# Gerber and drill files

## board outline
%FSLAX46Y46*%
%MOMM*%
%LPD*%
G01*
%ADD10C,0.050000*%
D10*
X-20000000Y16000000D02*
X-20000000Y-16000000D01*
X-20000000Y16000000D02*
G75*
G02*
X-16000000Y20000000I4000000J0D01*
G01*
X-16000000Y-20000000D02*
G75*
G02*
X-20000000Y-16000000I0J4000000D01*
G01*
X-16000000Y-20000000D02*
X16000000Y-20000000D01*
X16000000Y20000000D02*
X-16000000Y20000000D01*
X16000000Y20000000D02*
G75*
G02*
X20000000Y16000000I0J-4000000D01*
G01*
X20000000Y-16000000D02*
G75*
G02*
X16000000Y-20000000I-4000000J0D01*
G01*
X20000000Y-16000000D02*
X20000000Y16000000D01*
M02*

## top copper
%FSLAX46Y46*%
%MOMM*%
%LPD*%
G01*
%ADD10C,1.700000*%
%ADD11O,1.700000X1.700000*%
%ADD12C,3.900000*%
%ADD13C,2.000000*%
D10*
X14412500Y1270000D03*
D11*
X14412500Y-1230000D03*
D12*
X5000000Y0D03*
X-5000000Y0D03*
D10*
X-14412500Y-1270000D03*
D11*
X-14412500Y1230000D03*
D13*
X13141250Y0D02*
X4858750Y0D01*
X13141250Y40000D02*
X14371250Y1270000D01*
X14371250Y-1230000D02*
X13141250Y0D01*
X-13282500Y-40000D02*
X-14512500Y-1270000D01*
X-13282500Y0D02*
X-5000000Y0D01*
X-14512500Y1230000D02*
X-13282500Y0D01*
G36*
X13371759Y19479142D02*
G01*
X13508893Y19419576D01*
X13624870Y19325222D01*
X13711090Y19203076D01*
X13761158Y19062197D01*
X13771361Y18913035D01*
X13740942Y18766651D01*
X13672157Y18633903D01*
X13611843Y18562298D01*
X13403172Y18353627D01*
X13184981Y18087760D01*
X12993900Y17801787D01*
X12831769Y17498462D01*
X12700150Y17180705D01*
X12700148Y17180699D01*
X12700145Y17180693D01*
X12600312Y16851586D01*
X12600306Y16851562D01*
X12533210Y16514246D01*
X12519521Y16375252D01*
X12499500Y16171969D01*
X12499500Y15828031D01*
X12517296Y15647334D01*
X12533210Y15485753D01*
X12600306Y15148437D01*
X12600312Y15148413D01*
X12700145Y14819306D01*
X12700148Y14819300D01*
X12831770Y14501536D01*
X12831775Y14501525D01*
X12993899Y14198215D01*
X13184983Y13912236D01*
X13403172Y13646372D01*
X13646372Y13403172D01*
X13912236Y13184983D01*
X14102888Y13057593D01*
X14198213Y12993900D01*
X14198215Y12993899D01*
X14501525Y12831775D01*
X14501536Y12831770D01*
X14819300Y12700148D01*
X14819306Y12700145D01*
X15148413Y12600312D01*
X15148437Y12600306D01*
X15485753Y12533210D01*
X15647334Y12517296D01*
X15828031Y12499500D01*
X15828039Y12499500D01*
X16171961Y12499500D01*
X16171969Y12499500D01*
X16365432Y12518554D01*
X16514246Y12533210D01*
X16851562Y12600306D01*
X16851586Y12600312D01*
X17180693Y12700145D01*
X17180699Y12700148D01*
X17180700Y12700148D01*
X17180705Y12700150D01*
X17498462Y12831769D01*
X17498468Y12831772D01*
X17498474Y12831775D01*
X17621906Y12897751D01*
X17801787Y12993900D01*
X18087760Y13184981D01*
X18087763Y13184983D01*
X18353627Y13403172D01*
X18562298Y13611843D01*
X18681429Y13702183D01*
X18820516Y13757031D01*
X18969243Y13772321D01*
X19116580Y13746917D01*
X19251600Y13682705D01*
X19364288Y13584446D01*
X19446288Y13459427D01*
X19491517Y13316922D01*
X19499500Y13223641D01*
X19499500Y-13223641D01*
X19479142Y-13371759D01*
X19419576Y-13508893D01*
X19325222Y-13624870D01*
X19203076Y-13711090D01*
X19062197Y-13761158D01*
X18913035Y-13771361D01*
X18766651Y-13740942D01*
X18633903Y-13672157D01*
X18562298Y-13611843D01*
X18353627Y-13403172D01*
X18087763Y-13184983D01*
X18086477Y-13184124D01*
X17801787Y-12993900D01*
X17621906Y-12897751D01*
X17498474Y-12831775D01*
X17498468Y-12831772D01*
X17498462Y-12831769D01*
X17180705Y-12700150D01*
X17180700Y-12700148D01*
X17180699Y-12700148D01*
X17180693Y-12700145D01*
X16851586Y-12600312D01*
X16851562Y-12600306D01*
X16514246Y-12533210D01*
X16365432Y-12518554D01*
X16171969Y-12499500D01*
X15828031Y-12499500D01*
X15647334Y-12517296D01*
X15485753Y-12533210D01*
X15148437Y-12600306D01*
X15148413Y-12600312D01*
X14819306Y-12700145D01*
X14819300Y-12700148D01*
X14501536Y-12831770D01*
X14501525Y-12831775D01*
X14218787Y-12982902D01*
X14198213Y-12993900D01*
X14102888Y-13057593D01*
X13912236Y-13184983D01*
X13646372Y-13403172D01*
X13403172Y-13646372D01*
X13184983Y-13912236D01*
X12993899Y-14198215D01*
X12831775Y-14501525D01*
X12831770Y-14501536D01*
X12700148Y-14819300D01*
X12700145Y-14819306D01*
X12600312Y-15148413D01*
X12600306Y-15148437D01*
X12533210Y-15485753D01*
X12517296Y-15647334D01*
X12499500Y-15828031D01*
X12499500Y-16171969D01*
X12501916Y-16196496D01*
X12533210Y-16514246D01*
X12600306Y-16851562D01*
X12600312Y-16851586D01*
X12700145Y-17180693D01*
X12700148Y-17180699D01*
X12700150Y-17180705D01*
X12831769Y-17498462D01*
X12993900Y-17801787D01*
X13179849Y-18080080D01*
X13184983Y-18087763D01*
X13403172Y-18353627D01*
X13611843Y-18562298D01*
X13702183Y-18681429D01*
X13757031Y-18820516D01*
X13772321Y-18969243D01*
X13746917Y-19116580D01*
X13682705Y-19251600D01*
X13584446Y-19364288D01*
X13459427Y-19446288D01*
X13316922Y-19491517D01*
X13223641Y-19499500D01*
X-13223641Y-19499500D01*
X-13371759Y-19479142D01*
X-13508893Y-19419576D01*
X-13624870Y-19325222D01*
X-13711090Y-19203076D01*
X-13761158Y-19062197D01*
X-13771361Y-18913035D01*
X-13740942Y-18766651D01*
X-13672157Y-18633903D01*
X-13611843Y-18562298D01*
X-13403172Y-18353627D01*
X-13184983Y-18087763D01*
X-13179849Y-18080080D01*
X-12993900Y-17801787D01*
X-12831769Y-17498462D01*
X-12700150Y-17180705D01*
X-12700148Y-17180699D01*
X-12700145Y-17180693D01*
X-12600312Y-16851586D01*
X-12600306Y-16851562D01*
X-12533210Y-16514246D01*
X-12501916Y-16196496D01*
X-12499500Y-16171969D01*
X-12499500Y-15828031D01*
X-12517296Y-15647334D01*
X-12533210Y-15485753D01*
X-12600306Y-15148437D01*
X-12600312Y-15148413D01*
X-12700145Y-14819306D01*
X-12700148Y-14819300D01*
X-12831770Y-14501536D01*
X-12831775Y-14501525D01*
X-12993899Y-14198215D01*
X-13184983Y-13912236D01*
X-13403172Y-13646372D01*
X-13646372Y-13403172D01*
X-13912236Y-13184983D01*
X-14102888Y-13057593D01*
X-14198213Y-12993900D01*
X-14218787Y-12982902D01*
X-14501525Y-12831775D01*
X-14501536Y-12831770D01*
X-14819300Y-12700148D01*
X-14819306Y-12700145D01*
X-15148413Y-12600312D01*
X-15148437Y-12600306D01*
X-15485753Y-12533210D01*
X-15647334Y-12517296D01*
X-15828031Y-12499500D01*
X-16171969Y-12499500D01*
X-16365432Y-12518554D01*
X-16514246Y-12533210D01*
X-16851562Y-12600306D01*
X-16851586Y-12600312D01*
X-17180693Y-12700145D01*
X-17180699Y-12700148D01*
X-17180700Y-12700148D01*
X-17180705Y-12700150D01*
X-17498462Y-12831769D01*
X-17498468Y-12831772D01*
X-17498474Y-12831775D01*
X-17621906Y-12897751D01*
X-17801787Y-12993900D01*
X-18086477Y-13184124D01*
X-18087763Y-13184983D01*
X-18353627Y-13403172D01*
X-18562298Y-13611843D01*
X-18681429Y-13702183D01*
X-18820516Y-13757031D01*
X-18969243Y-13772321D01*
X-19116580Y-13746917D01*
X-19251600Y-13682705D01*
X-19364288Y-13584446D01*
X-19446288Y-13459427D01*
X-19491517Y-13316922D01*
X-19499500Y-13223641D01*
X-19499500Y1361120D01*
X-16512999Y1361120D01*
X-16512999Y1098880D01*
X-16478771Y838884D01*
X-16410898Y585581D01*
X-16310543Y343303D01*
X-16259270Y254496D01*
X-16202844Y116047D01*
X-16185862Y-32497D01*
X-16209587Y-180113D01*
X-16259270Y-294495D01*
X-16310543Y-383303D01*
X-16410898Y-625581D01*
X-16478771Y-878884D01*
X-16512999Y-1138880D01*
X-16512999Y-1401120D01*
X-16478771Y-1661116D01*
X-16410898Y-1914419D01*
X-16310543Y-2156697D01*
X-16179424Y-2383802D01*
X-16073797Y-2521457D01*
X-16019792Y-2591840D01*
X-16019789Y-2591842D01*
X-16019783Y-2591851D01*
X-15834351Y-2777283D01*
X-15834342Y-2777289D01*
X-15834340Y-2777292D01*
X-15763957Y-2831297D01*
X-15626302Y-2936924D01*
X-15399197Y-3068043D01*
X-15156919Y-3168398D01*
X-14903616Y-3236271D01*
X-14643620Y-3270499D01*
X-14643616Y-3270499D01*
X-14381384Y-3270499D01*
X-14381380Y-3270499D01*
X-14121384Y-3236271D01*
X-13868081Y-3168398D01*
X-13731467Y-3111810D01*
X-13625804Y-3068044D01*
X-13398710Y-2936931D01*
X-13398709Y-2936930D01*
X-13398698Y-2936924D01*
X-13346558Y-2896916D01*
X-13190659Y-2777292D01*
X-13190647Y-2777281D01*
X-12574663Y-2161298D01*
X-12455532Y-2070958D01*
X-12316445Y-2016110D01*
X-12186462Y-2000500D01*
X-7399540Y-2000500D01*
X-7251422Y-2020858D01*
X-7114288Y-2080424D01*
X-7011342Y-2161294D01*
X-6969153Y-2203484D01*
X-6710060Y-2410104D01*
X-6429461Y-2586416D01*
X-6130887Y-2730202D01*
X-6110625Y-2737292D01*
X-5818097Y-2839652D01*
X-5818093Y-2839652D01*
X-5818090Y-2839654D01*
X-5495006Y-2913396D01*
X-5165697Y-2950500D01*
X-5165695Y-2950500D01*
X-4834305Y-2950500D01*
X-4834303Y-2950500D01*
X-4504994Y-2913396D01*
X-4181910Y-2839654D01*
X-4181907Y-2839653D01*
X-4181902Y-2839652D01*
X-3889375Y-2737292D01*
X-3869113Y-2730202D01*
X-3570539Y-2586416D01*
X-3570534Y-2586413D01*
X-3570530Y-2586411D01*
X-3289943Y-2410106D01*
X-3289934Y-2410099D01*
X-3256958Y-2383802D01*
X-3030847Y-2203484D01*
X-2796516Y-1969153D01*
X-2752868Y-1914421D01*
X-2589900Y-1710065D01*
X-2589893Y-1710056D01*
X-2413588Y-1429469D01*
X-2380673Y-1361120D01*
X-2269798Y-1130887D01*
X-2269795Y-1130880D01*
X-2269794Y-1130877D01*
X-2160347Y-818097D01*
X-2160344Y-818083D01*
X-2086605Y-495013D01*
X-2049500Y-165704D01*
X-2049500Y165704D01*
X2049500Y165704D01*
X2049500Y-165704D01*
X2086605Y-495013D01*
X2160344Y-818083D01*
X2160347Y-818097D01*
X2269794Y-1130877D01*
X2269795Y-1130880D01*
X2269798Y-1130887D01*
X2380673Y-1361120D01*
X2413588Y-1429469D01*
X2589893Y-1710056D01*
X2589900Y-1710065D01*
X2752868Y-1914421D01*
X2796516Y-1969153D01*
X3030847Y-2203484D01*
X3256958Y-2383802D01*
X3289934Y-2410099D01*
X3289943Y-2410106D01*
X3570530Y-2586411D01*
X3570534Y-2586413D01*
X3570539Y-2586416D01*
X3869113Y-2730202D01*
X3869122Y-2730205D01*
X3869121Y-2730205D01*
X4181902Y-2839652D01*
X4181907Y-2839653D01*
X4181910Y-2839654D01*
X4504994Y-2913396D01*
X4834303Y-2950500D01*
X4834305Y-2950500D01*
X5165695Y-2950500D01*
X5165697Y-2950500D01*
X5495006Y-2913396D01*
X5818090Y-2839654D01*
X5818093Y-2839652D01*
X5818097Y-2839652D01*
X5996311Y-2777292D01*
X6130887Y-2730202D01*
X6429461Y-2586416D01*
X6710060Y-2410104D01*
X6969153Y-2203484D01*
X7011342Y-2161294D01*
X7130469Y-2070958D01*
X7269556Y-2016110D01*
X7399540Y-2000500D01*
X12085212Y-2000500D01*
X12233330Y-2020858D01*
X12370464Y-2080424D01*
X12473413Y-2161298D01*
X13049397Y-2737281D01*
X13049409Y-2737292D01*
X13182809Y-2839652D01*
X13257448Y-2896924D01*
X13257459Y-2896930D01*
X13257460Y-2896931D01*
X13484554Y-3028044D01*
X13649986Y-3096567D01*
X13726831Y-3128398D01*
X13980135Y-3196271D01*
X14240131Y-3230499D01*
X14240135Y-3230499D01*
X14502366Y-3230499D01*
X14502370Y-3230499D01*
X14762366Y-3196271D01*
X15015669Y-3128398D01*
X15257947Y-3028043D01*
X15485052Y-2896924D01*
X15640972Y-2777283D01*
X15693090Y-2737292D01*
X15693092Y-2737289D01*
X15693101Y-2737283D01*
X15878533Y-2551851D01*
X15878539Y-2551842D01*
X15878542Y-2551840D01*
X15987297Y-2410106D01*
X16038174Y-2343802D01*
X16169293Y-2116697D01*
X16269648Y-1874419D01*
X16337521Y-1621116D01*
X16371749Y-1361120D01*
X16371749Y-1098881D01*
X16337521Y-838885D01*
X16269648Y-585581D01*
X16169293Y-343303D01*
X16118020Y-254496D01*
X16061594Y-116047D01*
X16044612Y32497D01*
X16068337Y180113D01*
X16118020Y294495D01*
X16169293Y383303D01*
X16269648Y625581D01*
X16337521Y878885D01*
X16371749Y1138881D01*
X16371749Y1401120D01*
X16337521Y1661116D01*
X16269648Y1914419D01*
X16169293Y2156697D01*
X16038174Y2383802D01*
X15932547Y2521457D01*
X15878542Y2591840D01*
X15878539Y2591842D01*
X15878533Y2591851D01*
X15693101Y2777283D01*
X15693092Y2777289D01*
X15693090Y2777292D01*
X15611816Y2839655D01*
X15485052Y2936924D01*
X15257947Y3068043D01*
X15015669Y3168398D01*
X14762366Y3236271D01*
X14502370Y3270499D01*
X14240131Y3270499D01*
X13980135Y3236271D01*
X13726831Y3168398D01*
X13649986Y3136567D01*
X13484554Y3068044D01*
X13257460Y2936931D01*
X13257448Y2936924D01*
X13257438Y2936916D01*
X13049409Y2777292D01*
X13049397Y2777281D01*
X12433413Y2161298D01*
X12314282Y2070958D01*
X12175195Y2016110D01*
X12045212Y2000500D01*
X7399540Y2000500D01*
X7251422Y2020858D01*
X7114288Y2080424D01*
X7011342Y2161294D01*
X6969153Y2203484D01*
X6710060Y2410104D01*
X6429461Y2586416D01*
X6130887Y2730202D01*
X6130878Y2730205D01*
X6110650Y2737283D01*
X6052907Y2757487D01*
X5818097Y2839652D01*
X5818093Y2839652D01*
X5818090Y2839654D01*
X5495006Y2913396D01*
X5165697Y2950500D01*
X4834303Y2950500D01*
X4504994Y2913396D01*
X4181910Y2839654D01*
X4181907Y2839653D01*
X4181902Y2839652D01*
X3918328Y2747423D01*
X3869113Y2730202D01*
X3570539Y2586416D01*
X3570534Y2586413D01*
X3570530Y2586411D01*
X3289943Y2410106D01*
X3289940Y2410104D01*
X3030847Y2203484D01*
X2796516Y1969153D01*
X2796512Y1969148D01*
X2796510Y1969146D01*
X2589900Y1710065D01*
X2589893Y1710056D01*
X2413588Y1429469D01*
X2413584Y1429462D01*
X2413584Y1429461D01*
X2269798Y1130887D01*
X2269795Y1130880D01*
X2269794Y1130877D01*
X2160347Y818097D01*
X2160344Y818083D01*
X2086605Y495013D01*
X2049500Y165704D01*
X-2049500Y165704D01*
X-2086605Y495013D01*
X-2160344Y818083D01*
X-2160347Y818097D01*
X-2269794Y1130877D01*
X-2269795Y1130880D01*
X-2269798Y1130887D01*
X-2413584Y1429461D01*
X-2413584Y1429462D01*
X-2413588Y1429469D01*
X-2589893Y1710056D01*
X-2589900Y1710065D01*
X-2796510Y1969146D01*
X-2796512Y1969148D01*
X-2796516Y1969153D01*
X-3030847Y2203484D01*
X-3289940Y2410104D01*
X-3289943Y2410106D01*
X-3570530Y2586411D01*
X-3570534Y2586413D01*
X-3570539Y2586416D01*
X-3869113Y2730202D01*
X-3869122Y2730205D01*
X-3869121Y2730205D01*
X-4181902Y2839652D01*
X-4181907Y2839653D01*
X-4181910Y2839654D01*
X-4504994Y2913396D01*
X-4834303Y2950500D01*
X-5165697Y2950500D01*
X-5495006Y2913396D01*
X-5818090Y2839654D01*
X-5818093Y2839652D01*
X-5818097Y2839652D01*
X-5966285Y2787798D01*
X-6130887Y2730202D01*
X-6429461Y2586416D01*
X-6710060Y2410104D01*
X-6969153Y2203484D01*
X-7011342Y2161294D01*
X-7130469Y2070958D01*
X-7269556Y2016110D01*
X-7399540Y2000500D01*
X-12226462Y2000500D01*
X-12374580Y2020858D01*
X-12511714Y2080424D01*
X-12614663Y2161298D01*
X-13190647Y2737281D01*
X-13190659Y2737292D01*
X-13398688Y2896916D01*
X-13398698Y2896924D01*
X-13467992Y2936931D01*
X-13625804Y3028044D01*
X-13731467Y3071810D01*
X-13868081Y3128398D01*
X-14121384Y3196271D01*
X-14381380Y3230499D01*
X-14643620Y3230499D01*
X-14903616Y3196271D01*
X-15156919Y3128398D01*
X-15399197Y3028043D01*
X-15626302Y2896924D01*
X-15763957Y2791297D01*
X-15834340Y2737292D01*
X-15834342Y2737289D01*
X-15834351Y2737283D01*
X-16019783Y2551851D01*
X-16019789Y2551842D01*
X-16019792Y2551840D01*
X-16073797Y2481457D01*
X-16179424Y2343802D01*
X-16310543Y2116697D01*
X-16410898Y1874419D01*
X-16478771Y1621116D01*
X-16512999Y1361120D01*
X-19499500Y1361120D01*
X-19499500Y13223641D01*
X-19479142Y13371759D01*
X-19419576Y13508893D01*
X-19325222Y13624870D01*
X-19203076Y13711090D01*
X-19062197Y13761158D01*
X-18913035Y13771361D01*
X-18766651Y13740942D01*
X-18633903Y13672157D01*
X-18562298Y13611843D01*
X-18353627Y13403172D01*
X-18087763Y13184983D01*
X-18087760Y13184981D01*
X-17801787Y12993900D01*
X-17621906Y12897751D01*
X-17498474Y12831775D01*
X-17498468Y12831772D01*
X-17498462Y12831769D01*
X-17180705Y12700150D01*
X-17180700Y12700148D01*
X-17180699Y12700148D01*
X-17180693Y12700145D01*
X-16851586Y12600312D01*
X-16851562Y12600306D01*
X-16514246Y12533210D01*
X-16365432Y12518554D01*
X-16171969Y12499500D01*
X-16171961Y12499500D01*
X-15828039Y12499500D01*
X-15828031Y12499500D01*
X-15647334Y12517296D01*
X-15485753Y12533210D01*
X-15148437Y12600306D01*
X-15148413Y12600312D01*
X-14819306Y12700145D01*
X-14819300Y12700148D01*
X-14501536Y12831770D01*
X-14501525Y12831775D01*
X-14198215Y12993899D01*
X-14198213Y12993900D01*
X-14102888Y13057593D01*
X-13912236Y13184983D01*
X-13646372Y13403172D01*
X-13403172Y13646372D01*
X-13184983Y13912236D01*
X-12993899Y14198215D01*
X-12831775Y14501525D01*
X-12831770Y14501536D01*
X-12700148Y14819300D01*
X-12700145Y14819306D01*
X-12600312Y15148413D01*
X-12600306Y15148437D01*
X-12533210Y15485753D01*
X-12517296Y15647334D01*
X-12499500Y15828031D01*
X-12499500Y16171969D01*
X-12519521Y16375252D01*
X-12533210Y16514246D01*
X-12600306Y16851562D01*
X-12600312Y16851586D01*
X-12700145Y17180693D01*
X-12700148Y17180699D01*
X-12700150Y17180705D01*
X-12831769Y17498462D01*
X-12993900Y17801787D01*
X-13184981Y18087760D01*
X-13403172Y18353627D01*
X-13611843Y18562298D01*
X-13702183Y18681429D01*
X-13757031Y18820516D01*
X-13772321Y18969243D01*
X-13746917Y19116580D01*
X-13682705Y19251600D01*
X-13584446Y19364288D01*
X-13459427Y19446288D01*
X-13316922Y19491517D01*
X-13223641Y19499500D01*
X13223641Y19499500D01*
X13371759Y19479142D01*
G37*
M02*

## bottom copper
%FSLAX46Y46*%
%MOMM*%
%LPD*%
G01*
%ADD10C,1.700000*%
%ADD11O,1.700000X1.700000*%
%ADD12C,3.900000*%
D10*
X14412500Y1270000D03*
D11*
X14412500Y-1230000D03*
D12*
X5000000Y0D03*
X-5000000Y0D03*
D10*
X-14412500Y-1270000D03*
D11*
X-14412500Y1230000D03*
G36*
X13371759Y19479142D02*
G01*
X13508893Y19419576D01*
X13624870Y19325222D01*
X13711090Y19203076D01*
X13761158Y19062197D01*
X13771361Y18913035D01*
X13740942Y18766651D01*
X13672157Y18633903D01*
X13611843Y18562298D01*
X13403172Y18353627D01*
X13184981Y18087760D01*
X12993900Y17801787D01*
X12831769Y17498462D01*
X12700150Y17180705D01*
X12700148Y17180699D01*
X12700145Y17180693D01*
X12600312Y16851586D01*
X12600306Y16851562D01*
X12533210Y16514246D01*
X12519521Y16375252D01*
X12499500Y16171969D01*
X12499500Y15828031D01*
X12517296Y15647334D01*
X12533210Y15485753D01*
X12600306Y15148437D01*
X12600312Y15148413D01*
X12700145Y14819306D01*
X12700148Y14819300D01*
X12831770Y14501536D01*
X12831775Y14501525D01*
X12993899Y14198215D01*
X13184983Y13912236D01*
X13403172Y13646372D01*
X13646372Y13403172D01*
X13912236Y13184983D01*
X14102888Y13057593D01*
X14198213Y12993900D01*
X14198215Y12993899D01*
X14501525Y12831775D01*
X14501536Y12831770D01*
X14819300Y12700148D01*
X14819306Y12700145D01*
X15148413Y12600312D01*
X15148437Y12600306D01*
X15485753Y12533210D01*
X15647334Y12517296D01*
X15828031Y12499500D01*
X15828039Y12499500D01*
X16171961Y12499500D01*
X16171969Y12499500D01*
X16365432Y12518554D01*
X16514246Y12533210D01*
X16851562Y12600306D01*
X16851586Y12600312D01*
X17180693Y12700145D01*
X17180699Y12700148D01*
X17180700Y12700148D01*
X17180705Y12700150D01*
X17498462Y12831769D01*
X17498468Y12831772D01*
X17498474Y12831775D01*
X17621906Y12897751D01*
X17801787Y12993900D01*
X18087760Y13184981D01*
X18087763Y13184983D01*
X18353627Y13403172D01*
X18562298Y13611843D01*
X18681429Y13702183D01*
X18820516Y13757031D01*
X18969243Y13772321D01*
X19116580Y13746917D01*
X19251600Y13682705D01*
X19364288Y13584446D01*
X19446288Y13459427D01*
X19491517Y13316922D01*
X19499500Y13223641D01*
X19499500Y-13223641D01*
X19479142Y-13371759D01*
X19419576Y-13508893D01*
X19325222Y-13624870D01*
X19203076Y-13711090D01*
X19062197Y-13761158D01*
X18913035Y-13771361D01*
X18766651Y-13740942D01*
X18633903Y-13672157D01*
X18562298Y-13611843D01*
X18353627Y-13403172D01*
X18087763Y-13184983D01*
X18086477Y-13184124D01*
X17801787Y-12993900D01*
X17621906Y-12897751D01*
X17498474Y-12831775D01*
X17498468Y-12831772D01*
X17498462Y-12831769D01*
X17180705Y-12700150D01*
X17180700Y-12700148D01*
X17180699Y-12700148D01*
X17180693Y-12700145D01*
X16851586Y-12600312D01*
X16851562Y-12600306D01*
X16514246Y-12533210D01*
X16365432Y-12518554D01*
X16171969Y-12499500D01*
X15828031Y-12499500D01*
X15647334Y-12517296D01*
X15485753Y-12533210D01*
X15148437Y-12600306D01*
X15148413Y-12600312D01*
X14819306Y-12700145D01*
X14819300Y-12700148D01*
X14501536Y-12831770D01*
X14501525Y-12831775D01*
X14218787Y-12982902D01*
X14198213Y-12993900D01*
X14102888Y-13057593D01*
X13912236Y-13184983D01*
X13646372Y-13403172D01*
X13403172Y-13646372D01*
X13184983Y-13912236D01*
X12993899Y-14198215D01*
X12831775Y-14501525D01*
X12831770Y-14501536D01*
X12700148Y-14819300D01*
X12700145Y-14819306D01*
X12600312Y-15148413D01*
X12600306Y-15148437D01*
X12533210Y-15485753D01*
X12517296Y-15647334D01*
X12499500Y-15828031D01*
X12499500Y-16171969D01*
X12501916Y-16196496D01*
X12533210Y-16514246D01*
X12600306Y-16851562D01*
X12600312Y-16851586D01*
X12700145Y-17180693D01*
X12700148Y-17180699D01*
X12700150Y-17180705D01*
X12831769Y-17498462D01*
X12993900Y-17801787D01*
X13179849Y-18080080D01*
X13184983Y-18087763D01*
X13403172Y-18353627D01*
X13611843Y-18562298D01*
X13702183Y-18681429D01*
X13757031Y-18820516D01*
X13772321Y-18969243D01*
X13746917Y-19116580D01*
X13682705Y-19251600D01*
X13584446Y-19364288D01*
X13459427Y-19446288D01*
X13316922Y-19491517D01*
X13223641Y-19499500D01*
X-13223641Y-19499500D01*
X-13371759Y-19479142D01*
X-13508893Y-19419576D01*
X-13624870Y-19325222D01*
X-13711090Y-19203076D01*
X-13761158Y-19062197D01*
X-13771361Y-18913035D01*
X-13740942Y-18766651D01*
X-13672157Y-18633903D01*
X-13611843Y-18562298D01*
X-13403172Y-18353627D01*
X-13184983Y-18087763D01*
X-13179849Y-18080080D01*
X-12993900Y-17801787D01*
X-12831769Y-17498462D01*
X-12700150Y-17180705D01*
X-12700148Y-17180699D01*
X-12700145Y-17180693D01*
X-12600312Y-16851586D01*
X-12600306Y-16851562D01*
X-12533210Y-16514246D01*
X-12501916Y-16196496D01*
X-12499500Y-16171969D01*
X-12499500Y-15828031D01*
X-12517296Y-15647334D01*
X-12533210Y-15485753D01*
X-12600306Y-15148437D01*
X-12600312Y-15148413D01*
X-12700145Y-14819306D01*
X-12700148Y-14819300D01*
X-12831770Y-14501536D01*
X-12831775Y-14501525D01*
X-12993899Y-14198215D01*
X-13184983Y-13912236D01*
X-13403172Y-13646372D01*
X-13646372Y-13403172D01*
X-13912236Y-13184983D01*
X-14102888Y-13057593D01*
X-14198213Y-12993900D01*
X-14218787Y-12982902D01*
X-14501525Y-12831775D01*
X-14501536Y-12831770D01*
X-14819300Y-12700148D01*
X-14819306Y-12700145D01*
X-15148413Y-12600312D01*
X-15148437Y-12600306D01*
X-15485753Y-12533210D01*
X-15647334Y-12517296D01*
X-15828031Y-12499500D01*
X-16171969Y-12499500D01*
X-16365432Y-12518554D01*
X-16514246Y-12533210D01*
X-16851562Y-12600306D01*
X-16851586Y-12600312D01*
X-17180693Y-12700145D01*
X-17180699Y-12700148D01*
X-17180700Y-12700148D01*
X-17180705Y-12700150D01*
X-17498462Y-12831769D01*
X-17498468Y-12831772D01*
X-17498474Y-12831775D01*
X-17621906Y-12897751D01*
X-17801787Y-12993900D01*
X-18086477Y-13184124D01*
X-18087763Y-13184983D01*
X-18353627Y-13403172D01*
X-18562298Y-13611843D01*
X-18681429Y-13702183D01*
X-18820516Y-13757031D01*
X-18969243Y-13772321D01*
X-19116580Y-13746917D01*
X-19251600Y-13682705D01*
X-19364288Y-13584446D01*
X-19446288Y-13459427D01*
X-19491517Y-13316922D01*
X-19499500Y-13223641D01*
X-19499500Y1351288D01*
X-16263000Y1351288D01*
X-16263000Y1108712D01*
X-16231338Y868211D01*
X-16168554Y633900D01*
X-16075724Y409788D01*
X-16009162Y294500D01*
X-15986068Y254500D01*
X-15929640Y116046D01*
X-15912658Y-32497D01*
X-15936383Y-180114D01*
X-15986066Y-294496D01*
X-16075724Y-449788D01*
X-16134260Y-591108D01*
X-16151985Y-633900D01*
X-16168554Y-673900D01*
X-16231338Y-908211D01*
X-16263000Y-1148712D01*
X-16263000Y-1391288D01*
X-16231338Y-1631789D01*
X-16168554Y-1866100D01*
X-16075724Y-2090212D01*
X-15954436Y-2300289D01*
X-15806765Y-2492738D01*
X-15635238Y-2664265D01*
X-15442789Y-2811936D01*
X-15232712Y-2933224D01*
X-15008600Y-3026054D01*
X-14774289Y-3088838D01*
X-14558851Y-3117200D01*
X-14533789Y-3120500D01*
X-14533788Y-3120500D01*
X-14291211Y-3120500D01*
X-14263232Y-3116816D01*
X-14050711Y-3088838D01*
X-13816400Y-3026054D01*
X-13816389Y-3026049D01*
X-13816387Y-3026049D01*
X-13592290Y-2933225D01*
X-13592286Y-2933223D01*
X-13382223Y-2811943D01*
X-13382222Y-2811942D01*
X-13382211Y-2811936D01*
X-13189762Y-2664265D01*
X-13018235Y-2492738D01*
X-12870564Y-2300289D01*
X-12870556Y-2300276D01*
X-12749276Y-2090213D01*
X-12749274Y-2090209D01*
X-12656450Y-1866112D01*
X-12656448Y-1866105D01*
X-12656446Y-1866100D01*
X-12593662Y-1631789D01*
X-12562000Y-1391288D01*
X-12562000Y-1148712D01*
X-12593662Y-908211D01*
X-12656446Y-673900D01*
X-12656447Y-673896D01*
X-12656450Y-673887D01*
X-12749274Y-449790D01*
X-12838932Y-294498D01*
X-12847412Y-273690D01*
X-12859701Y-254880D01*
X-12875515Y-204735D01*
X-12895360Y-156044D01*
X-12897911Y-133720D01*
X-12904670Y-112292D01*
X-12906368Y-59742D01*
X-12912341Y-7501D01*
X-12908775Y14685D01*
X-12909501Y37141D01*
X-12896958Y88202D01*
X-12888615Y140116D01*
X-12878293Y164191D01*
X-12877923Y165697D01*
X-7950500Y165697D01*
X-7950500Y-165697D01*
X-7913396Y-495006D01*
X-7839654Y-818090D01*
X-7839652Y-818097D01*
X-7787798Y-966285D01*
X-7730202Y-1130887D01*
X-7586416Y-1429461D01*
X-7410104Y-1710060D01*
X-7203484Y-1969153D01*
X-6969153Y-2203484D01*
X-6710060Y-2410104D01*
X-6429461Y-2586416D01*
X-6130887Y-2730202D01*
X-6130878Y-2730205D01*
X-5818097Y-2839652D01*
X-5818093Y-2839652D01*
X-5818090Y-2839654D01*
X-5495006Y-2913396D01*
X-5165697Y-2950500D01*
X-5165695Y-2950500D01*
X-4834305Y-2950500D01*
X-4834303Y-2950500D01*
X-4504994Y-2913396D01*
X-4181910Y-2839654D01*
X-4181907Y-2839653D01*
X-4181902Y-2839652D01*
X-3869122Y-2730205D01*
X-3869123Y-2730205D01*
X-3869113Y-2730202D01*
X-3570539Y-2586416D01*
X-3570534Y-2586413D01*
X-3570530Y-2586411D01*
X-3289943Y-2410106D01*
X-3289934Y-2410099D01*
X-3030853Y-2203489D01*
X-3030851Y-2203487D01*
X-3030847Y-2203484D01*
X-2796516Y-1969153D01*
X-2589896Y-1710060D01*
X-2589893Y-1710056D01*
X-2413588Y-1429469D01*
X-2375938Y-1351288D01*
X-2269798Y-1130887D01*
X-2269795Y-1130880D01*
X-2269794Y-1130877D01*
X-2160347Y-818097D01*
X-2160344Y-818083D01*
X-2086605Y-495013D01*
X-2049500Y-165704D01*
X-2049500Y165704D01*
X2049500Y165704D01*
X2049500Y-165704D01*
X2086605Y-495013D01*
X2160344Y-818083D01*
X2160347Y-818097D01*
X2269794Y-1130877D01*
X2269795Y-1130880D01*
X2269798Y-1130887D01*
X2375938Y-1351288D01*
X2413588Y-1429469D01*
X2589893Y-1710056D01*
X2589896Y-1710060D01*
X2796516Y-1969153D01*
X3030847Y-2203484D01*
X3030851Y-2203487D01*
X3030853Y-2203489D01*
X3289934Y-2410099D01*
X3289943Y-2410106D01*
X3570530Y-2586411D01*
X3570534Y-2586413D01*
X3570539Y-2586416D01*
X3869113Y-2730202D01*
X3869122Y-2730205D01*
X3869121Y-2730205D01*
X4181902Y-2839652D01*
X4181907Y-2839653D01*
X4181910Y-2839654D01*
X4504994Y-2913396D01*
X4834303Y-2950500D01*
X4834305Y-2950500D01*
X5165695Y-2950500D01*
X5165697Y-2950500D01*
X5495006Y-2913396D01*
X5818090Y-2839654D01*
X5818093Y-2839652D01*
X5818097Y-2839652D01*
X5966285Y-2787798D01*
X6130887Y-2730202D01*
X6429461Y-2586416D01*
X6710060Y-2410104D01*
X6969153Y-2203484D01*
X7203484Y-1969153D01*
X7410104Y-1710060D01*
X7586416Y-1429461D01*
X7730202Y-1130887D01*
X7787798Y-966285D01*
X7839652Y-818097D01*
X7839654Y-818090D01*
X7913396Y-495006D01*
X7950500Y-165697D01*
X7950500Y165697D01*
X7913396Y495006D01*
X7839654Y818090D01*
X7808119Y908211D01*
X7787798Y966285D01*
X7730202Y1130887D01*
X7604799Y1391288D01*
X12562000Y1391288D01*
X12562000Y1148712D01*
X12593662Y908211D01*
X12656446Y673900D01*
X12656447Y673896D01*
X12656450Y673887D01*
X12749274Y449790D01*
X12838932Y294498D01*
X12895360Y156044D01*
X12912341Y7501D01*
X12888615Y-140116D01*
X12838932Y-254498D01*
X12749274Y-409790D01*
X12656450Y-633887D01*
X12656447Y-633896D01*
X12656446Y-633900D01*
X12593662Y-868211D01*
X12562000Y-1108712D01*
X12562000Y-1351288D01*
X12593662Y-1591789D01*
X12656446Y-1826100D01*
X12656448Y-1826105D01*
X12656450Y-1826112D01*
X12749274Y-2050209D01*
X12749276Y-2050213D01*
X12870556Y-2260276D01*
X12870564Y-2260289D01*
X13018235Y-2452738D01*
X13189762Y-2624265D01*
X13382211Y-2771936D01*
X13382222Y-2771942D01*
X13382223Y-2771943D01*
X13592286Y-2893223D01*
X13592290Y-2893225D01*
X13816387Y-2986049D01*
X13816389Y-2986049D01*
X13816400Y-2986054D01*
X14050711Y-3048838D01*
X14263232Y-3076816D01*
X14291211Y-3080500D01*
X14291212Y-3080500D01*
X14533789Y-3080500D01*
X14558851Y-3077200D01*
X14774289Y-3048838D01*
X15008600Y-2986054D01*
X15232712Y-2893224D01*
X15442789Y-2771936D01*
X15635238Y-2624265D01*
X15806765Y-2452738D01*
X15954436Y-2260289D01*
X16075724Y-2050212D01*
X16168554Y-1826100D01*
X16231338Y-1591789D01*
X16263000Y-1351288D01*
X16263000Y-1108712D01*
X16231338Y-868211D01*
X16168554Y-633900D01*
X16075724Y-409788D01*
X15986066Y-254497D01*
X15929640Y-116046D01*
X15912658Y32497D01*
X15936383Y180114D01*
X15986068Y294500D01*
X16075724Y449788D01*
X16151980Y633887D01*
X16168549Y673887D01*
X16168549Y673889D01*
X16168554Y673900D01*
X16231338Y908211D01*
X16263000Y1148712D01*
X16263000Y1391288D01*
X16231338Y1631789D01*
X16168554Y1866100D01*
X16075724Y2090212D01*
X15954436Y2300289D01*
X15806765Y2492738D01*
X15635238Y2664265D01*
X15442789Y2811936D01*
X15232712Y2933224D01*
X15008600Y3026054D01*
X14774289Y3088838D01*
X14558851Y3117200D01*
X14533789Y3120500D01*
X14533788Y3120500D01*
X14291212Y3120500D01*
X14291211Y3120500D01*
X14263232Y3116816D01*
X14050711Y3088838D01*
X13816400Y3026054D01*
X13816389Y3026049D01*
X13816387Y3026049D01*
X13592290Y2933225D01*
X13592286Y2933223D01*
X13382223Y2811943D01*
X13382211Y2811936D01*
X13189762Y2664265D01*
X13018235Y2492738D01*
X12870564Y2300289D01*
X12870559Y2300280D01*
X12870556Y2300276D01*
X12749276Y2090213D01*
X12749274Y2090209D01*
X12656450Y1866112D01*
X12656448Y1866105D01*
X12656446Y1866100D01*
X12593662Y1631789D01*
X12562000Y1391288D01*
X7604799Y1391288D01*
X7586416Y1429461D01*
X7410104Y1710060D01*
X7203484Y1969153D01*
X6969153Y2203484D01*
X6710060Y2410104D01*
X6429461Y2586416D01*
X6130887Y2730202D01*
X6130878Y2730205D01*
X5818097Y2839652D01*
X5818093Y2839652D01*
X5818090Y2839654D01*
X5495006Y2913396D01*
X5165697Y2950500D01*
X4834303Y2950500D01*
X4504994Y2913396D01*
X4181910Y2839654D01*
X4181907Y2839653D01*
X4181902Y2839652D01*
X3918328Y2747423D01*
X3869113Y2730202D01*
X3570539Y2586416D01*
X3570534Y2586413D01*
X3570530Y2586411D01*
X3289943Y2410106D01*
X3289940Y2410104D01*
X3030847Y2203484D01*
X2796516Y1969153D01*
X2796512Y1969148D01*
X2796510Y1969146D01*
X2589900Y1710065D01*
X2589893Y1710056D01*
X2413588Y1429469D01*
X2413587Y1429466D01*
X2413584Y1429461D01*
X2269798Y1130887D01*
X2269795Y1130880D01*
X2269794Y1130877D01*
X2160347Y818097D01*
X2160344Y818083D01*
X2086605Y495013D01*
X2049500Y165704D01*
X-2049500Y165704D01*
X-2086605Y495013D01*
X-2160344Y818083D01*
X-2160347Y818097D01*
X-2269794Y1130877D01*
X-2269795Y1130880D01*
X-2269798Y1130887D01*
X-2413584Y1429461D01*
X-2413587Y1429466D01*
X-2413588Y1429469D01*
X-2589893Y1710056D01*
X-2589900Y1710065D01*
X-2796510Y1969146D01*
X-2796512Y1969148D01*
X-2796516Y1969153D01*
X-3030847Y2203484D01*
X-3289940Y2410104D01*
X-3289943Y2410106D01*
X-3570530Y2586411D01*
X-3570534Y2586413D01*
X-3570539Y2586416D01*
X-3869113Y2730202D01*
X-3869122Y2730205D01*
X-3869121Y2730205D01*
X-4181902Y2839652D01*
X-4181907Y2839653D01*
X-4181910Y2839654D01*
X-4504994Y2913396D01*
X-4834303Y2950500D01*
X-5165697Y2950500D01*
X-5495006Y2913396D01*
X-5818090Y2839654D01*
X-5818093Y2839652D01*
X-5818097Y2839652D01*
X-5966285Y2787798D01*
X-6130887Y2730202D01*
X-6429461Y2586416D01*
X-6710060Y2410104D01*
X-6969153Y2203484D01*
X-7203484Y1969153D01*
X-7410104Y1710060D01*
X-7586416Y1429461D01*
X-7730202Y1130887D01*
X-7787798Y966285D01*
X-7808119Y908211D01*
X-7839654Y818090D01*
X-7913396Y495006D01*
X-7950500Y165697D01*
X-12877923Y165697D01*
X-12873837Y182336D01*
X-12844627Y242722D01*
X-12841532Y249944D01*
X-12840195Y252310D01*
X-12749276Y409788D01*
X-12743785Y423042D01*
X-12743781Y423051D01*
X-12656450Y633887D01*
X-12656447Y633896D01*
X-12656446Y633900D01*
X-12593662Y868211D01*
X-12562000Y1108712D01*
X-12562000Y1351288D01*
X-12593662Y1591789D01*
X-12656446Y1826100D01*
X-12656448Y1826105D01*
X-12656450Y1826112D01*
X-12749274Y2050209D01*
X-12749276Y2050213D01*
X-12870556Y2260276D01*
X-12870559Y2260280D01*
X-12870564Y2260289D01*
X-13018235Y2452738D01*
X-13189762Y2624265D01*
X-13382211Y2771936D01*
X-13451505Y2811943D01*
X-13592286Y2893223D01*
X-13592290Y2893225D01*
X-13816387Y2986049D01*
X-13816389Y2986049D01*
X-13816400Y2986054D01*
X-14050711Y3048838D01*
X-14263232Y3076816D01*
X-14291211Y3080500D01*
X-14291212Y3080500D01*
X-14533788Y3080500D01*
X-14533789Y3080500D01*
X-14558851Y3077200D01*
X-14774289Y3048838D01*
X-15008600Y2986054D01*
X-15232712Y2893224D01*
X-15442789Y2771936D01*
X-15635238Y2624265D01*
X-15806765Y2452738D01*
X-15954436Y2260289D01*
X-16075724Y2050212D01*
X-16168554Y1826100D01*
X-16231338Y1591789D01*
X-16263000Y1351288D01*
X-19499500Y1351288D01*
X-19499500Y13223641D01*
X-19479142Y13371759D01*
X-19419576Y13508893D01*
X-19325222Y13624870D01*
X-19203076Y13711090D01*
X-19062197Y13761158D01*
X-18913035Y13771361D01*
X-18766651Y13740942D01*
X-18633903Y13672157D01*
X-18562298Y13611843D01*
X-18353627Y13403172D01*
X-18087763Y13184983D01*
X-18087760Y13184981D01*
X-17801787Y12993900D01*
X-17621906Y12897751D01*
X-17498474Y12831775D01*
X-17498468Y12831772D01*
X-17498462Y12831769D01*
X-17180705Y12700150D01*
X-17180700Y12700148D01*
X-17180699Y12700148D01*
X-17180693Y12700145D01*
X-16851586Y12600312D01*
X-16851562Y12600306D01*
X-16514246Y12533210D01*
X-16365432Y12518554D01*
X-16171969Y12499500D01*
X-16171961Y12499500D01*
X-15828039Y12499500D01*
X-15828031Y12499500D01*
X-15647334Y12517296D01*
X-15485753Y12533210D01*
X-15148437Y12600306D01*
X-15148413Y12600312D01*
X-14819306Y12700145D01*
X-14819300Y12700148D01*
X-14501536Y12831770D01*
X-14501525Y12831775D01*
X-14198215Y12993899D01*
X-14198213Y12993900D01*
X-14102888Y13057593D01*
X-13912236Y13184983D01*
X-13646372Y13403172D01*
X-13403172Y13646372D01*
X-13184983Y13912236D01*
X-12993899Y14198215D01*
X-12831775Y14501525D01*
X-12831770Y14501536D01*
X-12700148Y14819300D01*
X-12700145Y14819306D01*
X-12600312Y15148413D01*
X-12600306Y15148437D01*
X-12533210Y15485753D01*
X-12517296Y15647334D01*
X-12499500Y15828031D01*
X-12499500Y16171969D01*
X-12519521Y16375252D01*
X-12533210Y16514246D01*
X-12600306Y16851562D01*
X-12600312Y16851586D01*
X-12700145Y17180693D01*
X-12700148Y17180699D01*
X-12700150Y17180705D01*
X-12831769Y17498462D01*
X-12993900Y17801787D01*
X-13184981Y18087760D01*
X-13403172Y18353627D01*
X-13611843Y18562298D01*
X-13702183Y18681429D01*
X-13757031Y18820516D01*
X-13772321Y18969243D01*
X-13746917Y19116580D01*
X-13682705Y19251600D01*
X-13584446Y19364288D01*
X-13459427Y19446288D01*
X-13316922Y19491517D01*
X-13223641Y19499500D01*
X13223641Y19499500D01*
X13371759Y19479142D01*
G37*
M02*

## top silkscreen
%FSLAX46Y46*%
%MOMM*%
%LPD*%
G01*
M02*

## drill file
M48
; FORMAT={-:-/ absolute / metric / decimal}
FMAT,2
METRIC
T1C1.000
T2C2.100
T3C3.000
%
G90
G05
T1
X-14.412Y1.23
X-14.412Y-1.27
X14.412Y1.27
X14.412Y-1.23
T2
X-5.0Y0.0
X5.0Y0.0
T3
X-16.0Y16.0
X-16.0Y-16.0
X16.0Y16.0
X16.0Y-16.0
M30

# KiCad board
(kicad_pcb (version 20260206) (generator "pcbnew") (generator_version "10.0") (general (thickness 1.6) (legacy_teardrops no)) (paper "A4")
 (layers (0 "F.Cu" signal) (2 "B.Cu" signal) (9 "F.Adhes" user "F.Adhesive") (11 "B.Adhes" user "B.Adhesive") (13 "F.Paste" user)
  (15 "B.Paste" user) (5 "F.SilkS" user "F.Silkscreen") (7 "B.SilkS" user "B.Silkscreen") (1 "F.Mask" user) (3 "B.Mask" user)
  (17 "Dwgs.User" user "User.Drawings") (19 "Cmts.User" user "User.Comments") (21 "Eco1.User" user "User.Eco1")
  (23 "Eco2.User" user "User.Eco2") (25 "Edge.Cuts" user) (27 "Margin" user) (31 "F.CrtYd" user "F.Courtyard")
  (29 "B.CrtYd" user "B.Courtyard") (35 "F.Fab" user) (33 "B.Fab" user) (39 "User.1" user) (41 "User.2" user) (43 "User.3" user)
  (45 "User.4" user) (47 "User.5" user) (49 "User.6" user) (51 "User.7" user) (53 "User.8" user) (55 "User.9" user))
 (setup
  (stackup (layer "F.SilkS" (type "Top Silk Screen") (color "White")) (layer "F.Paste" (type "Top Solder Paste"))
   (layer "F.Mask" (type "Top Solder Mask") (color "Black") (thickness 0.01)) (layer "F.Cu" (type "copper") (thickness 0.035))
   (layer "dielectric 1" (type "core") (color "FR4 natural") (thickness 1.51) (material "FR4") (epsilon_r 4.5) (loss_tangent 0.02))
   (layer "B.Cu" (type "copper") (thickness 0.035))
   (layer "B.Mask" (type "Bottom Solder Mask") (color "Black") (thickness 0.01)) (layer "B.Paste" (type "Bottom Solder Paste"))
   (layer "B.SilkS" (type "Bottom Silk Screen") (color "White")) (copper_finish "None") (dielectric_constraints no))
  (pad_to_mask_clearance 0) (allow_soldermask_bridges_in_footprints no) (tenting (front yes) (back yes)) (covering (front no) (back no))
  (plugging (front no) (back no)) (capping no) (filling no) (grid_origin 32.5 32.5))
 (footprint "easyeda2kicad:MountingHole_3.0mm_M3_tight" (layer "F.Cu") (at 16 -16 -90)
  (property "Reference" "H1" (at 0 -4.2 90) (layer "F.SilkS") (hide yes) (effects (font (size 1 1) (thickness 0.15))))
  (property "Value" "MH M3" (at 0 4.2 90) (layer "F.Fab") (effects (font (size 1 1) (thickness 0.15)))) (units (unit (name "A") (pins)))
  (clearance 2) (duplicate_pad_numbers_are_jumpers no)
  (pad "" np_thru_hole circle (at 0 0 270) (size 3 3) (drill 3) (layers "*.Cu" "*.Mask")))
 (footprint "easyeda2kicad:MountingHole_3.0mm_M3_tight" (layer "F.Cu") (at 16 16 -90)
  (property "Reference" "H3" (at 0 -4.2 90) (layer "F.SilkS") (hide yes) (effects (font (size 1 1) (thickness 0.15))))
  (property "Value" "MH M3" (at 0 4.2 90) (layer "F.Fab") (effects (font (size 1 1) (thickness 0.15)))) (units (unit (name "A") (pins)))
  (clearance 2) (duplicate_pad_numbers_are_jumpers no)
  (pad "" np_thru_hole circle (at 0 0 270) (size 3 3) (drill 3) (layers "*.Cu" "*.Mask")))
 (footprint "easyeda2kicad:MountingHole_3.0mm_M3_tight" (layer "F.Cu") (at -16 -16 -90)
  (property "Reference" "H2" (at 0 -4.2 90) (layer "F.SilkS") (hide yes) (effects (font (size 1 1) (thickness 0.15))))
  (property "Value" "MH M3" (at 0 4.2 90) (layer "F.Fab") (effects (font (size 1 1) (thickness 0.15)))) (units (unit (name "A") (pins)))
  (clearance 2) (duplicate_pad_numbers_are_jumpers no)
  (pad "" np_thru_hole circle (at 0 0 270) (size 3 3) (drill 3) (layers "*.Cu" "*.Mask")))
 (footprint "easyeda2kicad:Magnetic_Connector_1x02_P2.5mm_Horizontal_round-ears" (layer "F.Cu") (at 14.5125 0)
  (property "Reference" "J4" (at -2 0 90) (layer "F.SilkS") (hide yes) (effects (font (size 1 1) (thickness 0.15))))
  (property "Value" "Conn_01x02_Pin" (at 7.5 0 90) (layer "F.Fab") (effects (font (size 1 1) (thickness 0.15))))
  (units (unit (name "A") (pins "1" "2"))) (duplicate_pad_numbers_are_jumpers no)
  (pad "1" thru_hole circle (at -0.1 -1.27) (size 1.7 1.7) (drill 1) (layers "*.Cu" "*.Mask") (remove_unused_layers no)
   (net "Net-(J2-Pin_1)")
   (teardrops (best_length_ratio 0.5) (max_length 1) (best_width_ratio 1) (max_width 2) (curved_edges yes) (filter_ratio 0.9) (enabled yes)
    (allow_two_segments yes) (prefer_zone_connections yes)))
  (pad "2" thru_hole oval (at -0.1 1.23) (size 1.7 1.7) (drill 1) (layers "*.Cu" "*.Mask") (remove_unused_layers no) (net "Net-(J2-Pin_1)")
   (teardrops (best_length_ratio 0.5) (max_length 1) (best_width_ratio 1) (max_width 2) (curved_edges yes) (filter_ratio 0.9) (enabled yes)
    (allow_two_segments yes) (prefer_zone_connections yes))))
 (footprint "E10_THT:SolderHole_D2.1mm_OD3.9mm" (layer "F.Cu") (at 5 0)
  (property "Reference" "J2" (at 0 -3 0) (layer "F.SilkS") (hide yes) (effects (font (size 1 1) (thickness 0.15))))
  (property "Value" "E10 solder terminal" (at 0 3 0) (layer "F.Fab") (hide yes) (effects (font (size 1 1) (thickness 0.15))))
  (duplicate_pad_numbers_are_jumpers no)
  (pad "1" thru_hole circle (at 0 0) (size 3.9 3.9) (drill 2.1) (layers "*.Cu" "*.Mask") (remove_unused_layers no) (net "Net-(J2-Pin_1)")))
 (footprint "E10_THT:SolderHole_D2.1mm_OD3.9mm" (layer "F.Cu") (at -5 0)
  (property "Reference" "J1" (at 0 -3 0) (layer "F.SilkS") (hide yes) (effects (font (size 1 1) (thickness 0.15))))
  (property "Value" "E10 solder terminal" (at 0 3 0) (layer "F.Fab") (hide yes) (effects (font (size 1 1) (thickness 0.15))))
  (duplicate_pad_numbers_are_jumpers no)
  (pad "1" thru_hole circle (at 0 0) (size 3.9 3.9) (drill 2.1) (layers "*.Cu" "*.Mask") (remove_unused_layers no) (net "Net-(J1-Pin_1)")))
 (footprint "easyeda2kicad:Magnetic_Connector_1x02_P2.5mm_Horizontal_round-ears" (layer "F.Cu") (at -14.5125 0 180)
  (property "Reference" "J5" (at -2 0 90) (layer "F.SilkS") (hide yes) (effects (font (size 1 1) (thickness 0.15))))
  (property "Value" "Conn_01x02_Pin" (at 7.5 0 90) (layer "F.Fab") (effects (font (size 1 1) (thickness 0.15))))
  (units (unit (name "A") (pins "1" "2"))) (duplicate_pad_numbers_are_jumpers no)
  (pad "1" thru_hole circle (at -0.1 -1.27 180) (size 1.7 1.7) (drill 1) (layers "*.Cu" "*.Mask") (remove_unused_layers no)
   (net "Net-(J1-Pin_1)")
   (teardrops (best_length_ratio 0.5) (max_length 1) (best_width_ratio 1) (max_width 2) (curved_edges yes) (filter_ratio 0.9) (enabled yes)
    (allow_two_segments yes) (prefer_zone_connections yes)))
  (pad "2" thru_hole oval (at -0.1 1.23 180) (size 1.7 1.7) (drill 1) (layers "*.Cu" "*.Mask") (remove_unused_layers no)
   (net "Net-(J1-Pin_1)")
   (teardrops (best_length_ratio 0.5) (max_length 1) (best_width_ratio 1) (max_width 2) (curved_edges yes) (filter_ratio 0.9) (enabled yes)
    (allow_two_segments yes) (prefer_zone_connections yes))))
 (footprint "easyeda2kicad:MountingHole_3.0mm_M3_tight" (layer "F.Cu") (at -16 16 -90)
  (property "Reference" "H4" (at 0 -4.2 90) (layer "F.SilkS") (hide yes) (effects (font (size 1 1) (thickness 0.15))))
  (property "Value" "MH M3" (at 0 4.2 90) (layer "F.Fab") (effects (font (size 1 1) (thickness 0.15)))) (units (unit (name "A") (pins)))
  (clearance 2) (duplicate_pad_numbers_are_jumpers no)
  (pad "" np_thru_hole circle (at 0 0 270) (size 3 3) (drill 3) (layers "*.Cu" "*.Mask")))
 (gr_line (start -20 -16) (end -20 16) (stroke (width 0.05) (type default)) (layer "Edge.Cuts"))
 (gr_arc (start -20 -16) (mid -18.828427 -18.828427) (end -16 -20) (stroke (width 0.05) (type default)) (layer "Edge.Cuts"))
 (gr_arc (start -16 20) (mid -18.828427 18.828427) (end -20 16) (stroke (width 0.05) (type default)) (layer "Edge.Cuts"))
 (gr_line (start -16 20) (end 16 20) (stroke (width 0.05) (type default)) (layer "Edge.Cuts"))
 (gr_line (start 16 -20) (end -16 -20) (stroke (width 0.05) (type default)) (layer "Edge.Cuts"))
 (gr_arc (start 16 -20) (mid 18.828427 -18.828427) (end 20 -16) (stroke (width 0.05) (type default)) (layer "Edge.Cuts"))
 (gr_arc (start 20 16) (mid 18.828427 18.828427) (end 16 20) (stroke (width 0.05) (type default)) (layer "Edge.Cuts"))
 (gr_line (start 20 16) (end 20 -16) (stroke (width 0.05) (type default)) (layer "Edge.Cuts"))
 (segment (start 13.14125 0) (end 4.85875 0) (width 2) (layer "F.Cu") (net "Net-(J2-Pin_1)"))
 (segment (start 13.14125 -0.04) (end 14.37125 -1.27) (width 2) (layer "F.Cu") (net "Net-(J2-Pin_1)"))
 (segment (start 14.37125 1.23) (end 13.14125 0) (width 2) (layer "F.Cu") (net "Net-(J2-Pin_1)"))
 (segment (start -13.2825 0.04) (end -14.5125 1.27) (width 2) (layer "F.Cu") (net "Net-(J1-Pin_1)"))
 (segment (start -13.2825 0) (end -5 0) (width 2) (layer "F.Cu") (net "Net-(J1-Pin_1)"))
 (segment (start -14.5125 -1.23) (end -13.2825 0) (width 2) (layer "F.Cu") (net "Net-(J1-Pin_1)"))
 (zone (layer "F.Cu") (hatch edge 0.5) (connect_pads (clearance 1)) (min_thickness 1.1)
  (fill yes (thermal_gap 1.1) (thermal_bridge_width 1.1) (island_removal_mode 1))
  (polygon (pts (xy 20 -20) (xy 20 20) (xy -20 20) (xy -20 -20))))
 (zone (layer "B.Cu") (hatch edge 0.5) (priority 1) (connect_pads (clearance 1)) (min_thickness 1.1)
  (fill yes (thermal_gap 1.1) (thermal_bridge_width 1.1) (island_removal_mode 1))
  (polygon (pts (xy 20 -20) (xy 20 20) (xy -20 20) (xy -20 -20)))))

